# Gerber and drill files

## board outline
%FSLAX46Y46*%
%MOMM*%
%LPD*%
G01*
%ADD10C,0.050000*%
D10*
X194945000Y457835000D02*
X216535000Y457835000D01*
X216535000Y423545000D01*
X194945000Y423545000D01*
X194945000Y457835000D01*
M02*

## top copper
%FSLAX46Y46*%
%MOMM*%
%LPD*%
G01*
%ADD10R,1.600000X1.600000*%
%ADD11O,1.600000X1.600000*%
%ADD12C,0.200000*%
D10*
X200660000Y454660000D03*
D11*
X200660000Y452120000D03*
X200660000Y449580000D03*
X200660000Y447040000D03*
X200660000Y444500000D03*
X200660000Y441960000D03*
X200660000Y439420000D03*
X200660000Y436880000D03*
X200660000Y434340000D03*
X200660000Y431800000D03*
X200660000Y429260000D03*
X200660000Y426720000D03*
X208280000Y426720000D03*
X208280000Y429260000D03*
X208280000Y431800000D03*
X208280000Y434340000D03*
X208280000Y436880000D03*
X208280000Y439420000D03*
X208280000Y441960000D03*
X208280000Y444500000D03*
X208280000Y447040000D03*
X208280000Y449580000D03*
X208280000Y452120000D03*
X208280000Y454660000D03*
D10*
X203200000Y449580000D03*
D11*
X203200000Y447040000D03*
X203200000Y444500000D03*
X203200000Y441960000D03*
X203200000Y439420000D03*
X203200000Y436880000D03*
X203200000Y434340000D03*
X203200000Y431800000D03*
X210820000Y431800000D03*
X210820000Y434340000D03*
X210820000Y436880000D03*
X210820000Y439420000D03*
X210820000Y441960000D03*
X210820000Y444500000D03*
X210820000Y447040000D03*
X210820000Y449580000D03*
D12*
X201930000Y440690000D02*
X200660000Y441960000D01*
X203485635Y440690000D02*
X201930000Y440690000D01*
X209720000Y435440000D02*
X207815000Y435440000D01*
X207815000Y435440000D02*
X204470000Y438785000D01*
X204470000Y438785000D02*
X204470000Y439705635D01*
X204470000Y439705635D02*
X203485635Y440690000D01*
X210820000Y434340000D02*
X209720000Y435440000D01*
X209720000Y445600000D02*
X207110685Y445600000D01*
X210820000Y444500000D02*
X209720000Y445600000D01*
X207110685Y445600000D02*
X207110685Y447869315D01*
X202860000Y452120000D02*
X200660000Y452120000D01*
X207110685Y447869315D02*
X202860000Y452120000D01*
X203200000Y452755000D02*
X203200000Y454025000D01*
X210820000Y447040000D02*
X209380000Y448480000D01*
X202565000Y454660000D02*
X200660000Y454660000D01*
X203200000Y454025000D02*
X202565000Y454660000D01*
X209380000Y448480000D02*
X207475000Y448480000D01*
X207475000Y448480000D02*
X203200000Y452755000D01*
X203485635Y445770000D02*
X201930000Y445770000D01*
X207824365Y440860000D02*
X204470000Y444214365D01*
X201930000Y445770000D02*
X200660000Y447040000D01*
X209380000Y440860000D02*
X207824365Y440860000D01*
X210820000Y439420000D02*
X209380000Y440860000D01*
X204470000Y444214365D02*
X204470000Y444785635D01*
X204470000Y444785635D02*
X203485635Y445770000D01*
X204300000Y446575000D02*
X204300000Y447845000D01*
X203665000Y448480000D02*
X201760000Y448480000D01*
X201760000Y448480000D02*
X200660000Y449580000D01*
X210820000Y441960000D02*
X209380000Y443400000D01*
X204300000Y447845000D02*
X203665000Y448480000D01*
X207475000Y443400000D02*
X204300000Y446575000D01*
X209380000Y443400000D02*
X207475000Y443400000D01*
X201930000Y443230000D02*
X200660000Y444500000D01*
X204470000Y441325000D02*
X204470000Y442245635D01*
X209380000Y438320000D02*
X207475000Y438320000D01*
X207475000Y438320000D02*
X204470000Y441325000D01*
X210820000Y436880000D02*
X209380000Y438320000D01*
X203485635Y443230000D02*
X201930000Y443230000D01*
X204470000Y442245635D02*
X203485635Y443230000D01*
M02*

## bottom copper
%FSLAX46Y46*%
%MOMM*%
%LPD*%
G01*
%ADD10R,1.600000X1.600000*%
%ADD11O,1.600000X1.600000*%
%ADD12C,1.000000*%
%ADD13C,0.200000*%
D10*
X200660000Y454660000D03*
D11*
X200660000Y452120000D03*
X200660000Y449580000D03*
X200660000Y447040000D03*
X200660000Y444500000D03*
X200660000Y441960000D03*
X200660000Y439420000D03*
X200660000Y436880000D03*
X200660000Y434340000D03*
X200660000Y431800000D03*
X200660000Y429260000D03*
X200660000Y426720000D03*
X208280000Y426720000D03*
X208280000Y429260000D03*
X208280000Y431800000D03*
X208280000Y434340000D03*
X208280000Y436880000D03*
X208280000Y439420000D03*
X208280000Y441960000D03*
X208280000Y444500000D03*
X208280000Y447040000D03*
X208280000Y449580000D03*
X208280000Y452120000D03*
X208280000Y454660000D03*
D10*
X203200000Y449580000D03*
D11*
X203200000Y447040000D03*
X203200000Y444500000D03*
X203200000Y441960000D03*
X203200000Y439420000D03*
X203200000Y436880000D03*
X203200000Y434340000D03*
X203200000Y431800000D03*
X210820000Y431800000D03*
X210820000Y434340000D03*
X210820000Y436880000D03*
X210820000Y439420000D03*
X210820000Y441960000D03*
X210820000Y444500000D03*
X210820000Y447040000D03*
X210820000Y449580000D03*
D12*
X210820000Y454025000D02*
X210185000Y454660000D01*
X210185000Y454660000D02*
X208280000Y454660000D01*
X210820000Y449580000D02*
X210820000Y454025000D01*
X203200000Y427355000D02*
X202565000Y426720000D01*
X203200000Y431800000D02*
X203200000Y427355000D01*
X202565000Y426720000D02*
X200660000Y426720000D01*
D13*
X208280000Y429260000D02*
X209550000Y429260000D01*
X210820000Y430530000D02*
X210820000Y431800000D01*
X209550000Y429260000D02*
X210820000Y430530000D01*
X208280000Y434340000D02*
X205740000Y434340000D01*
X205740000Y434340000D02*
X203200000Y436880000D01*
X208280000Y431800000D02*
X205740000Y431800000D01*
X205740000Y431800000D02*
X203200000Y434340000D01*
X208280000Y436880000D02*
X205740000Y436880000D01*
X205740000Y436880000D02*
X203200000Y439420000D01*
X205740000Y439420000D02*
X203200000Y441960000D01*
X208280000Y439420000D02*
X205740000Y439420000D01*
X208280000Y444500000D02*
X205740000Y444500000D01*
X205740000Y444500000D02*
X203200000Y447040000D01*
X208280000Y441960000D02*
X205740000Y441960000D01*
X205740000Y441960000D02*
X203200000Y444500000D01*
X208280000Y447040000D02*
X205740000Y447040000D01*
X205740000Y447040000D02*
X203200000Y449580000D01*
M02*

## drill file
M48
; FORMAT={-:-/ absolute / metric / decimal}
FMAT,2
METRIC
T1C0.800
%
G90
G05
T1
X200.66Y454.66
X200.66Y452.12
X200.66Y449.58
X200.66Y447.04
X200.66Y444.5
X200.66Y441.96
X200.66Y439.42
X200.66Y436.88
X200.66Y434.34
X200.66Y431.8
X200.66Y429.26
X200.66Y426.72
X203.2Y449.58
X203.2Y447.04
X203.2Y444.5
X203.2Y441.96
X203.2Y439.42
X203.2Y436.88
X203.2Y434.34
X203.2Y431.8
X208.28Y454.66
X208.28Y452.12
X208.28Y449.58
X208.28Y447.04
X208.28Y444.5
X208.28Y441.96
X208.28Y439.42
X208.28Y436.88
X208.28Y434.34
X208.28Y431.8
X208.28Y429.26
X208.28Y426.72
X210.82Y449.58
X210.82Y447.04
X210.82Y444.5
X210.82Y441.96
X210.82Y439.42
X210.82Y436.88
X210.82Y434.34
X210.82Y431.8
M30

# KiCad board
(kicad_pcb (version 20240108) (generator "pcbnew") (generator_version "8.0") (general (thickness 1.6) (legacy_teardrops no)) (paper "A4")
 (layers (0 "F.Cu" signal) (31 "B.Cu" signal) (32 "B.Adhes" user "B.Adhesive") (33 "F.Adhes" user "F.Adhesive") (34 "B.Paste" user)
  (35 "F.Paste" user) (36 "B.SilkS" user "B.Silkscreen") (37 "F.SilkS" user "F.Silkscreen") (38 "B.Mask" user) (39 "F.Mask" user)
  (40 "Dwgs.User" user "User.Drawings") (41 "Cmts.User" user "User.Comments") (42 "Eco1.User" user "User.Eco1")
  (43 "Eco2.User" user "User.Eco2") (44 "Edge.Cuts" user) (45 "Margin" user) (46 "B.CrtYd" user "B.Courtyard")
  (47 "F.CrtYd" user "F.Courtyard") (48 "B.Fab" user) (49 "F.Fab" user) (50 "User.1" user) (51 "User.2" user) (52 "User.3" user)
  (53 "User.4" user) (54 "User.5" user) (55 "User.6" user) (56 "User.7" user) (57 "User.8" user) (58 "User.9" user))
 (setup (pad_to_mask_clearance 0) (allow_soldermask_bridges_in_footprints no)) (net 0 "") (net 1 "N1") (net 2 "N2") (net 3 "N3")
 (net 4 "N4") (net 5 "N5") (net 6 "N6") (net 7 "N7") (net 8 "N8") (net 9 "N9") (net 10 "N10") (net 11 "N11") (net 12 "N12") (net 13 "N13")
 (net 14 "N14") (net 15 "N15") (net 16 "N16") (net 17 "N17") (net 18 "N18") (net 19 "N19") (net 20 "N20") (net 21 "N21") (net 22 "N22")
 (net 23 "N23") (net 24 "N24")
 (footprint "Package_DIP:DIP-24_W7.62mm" (layer "F.Cu") (at 200.66 -454.66)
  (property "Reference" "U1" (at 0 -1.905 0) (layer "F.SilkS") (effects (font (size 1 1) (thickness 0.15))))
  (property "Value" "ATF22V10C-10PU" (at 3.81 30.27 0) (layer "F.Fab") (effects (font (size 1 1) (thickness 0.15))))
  (pad "1" thru_hole rect (at 0 0) (size 1.6 1.6) (drill 0.8) (layers "*.Cu" "*.Mask") (remove_unused_layers no) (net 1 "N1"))
  (pad "2" thru_hole oval (at 0 2.54) (size 1.6 1.6) (drill 0.8) (layers "*.Cu" "*.Mask") (remove_unused_layers no) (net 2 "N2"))
  (pad "3" thru_hole oval (at 0 5.08) (size 1.6 1.6) (drill 0.8) (layers "*.Cu" "*.Mask") (remove_unused_layers no) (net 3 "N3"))
  (pad "4" thru_hole oval (at 0 7.62) (size 1.6 1.6) (drill 0.8) (layers "*.Cu" "*.Mask") (remove_unused_layers no) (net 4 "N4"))
  (pad "5" thru_hole oval (at 0 10.16) (size 1.6 1.6) (drill 0.8) (layers "*.Cu" "*.Mask") (remove_unused_layers no) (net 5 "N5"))
  (pad "6" thru_hole oval (at 0 12.7) (size 1.6 1.6) (drill 0.8) (layers "*.Cu" "*.Mask") (remove_unused_layers no) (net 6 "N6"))
  (pad "7" thru_hole oval (at 0 15.24) (size 1.6 1.6) (drill 0.8) (layers "*.Cu" "*.Mask") (remove_unused_layers no) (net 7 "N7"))
  (pad "8" thru_hole oval (at 0 17.78) (size 1.6 1.6) (drill 0.8) (layers "*.Cu" "*.Mask") (remove_unused_layers no) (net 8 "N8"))
  (pad "9" thru_hole oval (at 0 20.32) (size 1.6 1.6) (drill 0.8) (layers "*.Cu" "*.Mask") (remove_unused_layers no) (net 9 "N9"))
  (pad "10" thru_hole oval (at 0 22.86) (size 1.6 1.6) (drill 0.8) (layers "*.Cu" "*.Mask") (remove_unused_layers no) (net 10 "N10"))
  (pad "11" thru_hole oval (at 0 25.4) (size 1.6 1.6) (drill 0.8) (layers "*.Cu" "*.Mask") (remove_unused_layers no) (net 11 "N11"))
  (pad "12" thru_hole oval (at 0 27.94) (size 1.6 1.6) (drill 0.8) (layers "*.Cu" "*.Mask") (remove_unused_layers no) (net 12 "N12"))
  (pad "13" thru_hole oval (at 7.62 27.94) (size 1.6 1.6) (drill 0.8) (layers "*.Cu" "*.Mask") (remove_unused_layers no) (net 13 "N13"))
  (pad "14" thru_hole oval (at 7.62 25.4) (size 1.6 1.6) (drill 0.8) (layers "*.Cu" "*.Mask") (remove_unused_layers no) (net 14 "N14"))
  (pad "15" thru_hole oval (at 7.62 22.86) (size 1.6 1.6) (drill 0.8) (layers "*.Cu" "*.Mask") (remove_unused_layers no) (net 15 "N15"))
  (pad "16" thru_hole oval (at 7.62 20.32) (size 1.6 1.6) (drill 0.8) (layers "*.Cu" "*.Mask") (remove_unused_layers no) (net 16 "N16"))
  (pad "17" thru_hole oval (at 7.62 17.78) (size 1.6 1.6) (drill 0.8) (layers "*.Cu" "*.Mask") (remove_unused_layers no) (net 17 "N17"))
  (pad "18" thru_hole oval (at 7.62 15.24) (size 1.6 1.6) (drill 0.8) (layers "*.Cu" "*.Mask") (remove_unused_layers no) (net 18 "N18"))
  (pad "19" thru_hole oval (at 7.62 12.7) (size 1.6 1.6) (drill 0.8) (layers "*.Cu" "*.Mask") (remove_unused_layers no) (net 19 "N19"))
  (pad "20" thru_hole oval (at 7.62 10.16) (size 1.6 1.6) (drill 0.8) (layers "*.Cu" "*.Mask") (remove_unused_layers no) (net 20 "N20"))
  (pad "21" thru_hole oval (at 7.62 7.62) (size 1.6 1.6) (drill 0.8) (layers "*.Cu" "*.Mask") (remove_unused_layers no) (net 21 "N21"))
  (pad "22" thru_hole oval (at 7.62 5.08) (size 1.6 1.6) (drill 0.8) (layers "*.Cu" "*.Mask") (remove_unused_layers no) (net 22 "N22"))
  (pad "23" thru_hole oval (at 7.62 2.54) (size 1.6 1.6) (drill 0.8) (layers "*.Cu" "*.Mask") (remove_unused_layers no) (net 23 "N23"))
  (pad "24" thru_hole oval (at 7.62 0) (size 1.6 1.6) (drill 0.8) (layers "*.Cu" "*.Mask") (remove_unused_layers no) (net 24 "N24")))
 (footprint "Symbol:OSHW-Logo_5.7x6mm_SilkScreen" (layer "F.Cu") (at 212.725 -427.355 90)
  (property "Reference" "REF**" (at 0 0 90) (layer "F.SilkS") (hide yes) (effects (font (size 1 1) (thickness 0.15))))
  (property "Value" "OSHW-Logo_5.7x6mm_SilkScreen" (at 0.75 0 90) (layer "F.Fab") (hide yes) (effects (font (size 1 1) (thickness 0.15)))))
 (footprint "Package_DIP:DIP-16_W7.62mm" (layer "F.Cu") (at 203.2 -449.58)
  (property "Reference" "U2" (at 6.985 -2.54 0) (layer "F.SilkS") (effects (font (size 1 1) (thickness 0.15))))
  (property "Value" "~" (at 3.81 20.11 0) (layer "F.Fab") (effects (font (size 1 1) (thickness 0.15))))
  (pad "1" thru_hole rect (at 0 0) (size 1.6 1.6) (drill 0.8) (layers "*.Cu" "*.Mask") (remove_unused_layers no) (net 21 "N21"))
  (pad "2" thru_hole oval (at 0 2.54) (size 1.6 1.6) (drill 0.8) (layers "*.Cu" "*.Mask") (remove_unused_layers no) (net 20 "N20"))
  (pad "3" thru_hole oval (at 0 5.08) (size 1.6 1.6) (drill 0.8) (layers "*.Cu" "*.Mask") (remove_unused_layers no) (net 19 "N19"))
  (pad "4" thru_hole oval (at 0 7.62) (size 1.6 1.6) (drill 0.8) (layers "*.Cu" "*.Mask") (remove_unused_layers no) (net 18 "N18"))
  (pad "5" thru_hole oval (at 0 10.16) (size 1.6 1.6) (drill 0.8) (layers "*.Cu" "*.Mask") (remove_unused_layers no) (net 17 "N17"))
  (pad "6" thru_hole oval (at 0 12.7) (size 1.6 1.6) (drill 0.8) (layers "*.Cu" "*.Mask") (remove_unused_layers no) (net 16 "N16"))
  (pad "7" thru_hole oval (at 0 15.24) (size 1.6 1.6) (drill 0.8) (layers "*.Cu" "*.Mask") (remove_unused_layers no) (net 15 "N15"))
  (pad "8" thru_hole oval (at 0 17.78) (size 1.6 1.6) (drill 0.8) (layers "*.Cu" "*.Mask") (remove_unused_layers no) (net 12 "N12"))
  (pad "9" thru_hole oval (at 7.62 17.78) (size 1.6 1.6) (drill 0.8) (layers "*.Cu" "*.Mask") (remove_unused_layers no) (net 14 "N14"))
  (pad "10" thru_hole oval (at 7.62 15.24) (size 1.6 1.6) (drill 0.8) (layers "*.Cu" "*.Mask") (remove_unused_layers no) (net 6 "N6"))
  (pad "11" thru_hole oval (at 7.62 12.7) (size 1.6 1.6) (drill 0.8) (layers "*.Cu" "*.Mask") (remove_unused_layers no) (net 5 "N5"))
  (pad "12" thru_hole oval (at 7.62 10.16) (size 1.6 1.6) (drill 0.8) (layers "*.Cu" "*.Mask") (remove_unused_layers no) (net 4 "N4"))
  (pad "13" thru_hole oval (at 7.62 7.62) (size 1.6 1.6) (drill 0.8) (layers "*.Cu" "*.Mask") (remove_unused_layers no) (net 3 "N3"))
  (pad "14" thru_hole oval (at 7.62 5.08) (size 1.6 1.6) (drill 0.8) (layers "*.Cu" "*.Mask") (remove_unused_layers no) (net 2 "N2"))
  (pad "15" thru_hole oval (at 7.62 2.54) (size 1.6 1.6) (drill 0.8) (layers "*.Cu" "*.Mask") (remove_unused_layers no) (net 1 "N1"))
  (pad "16" thru_hole oval (at 7.62 0) (size 1.6 1.6) (drill 0.8) (layers "*.Cu" "*.Mask") (remove_unused_layers no) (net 24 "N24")))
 (gr_rect (start 194.945 -457.835) (end 216.535 -423.545) (stroke (width 0.05) (type default)) (fill none) (layer "Edge.Cuts"))
 (segment (start 210.82 -454.025) (end 210.185 -454.66) (width 1) (layer "B.Cu") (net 24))
 (segment (start 210.185 -454.66) (end 208.28 -454.66) (width 1) (layer "B.Cu") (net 24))
 (segment (start 210.82 -449.58) (end 210.82 -454.025) (width 1) (layer "B.Cu") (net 24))
 (segment (start 203.2 -427.355) (end 202.565 -426.72) (width 1) (layer "B.Cu") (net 12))
 (segment (start 203.2 -431.8) (end 203.2 -427.355) (width 1) (layer "B.Cu") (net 12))
 (segment (start 202.565 -426.72) (end 200.66 -426.72) (width 1) (layer "B.Cu") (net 12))
 (segment (start 208.28 -429.26) (end 209.55 -429.26) (width 0.2) (layer "B.Cu") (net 14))
 (segment (start 210.82 -430.53) (end 210.82 -431.8) (width 0.2) (layer "B.Cu") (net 14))
 (segment (start 209.55 -429.26) (end 210.82 -430.53) (width 0.2) (layer "B.Cu") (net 14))
 (segment (start 208.28 -434.34) (end 205.74 -434.34) (width 0.2) (layer "B.Cu") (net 16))
 (segment (start 205.74 -434.34) (end 203.2 -436.88) (width 0.2) (layer "B.Cu") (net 16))
 (segment (start 208.28 -431.8) (end 205.74 -431.8) (width 0.2) (layer "B.Cu") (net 15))
 (segment (start 205.74 -431.8) (end 203.2 -434.34) (width 0.2) (layer "B.Cu") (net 15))
 (segment (start 208.28 -436.88) (end 205.74 -436.88) (width 0.2) (layer "B.Cu") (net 17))
 (segment (start 205.74 -436.88) (end 203.2 -439.42) (width 0.2) (layer "B.Cu") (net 17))
 (segment (start 205.74 -439.42) (end 203.2 -441.96) (width 0.2) (layer "B.Cu") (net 18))
 (segment (start 208.28 -439.42) (end 205.74 -439.42) (width 0.2) (layer "B.Cu") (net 18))
 (segment (start 208.28 -444.5) (end 205.74 -444.5) (width 0.2) (layer "B.Cu") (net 20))
 (segment (start 205.74 -444.5) (end 203.2 -447.04) (width 0.2) (layer "B.Cu") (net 20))
 (segment (start 208.28 -441.96) (end 205.74 -441.96) (width 0.2) (layer "B.Cu") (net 19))
 (segment (start 205.74 -441.96) (end 203.2 -444.5) (width 0.2) (layer "B.Cu") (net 19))
 (segment (start 208.28 -447.04) (end 205.74 -447.04) (width 0.2) (layer "B.Cu") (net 21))
 (segment (start 205.74 -447.04) (end 203.2 -449.58) (width 0.2) (layer "B.Cu") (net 21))
 (segment (start 201.93 -440.69) (end 200.66 -441.96) (width 0.2) (layer "F.Cu") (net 6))
 (segment (start 203.485635 -440.69) (end 201.93 -440.69) (width 0.2) (layer "F.Cu") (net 6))
 (segment (start 209.72 -435.44) (end 207.815 -435.44) (width 0.2) (layer "F.Cu") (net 6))
 (segment (start 207.815 -435.44) (end 204.47 -438.785) (width 0.2) (layer "F.Cu") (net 6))
 (segment (start 204.47 -438.785) (end 204.47 -439.705635) (width 0.2) (layer "F.Cu") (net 6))
 (segment (start 204.47 -439.705635) (end 203.485635 -440.69) (width 0.2) (layer "F.Cu") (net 6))
 (segment (start 210.82 -434.34) (end 209.72 -435.44) (width 0.2) (layer "F.Cu") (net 6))
 (segment (start 209.72 -445.6) (end 207.110685 -445.6) (width 0.2) (layer "F.Cu") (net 2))
 (segment (start 210.82 -444.5) (end 209.72 -445.6) (width 0.2) (layer "F.Cu") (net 2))
 (segment (start 207.110685 -445.6) (end 207.110685 -447.869315) (width 0.2) (layer "F.Cu") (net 2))
 (segment (start 202.86 -452.12) (end 200.66 -452.12) (width 0.2) (layer "F.Cu") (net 2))
 (segment (start 207.110685 -447.869315) (end 202.86 -452.12) (width 0.2) (layer "F.Cu") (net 2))
 (segment (start 203.2 -452.755) (end 203.2 -454.025) (width 0.2) (layer "F.Cu") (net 1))
 (segment (start 210.82 -447.04) (end 209.38 -448.48) (width 0.2) (layer "F.Cu") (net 1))
 (segment (start 202.565 -454.66) (end 200.66 -454.66) (width 0.2) (layer "F.Cu") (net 1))
 (segment (start 203.2 -454.025) (end 202.565 -454.66) (width 0.2) (layer "F.Cu") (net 1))
 (segment (start 209.38 -448.48) (end 207.475 -448.48) (width 0.2) (layer "F.Cu") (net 1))
 (segment (start 207.475 -448.48) (end 203.2 -452.755) (width 0.2) (layer "F.Cu") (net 1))
 (segment (start 203.485635 -445.77) (end 201.93 -445.77) (width 0.2) (layer "F.Cu") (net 4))
 (segment (start 207.824365 -440.86) (end 204.47 -444.214365) (width 0.2) (layer "F.Cu") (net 4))
 (segment (start 201.93 -445.77) (end 200.66 -447.04) (width 0.2) (layer "F.Cu") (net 4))
 (segment (start 209.38 -440.86) (end 207.824365 -440.86) (width 0.2) (layer "F.Cu") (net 4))
 (segment (start 210.82 -439.42) (end 209.38 -440.86) (width 0.2) (layer "F.Cu") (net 4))
 (segment (start 204.47 -444.214365) (end 204.47 -444.785635) (width 0.2) (layer "F.Cu") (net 4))
 (segment (start 204.47 -444.785635) (end 203.485635 -445.77) (width 0.2) (layer "F.Cu") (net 4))
 (segment (start 204.3 -446.575) (end 204.3 -447.845) (width 0.2) (layer "F.Cu") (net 3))
 (segment (start 203.665 -448.48) (end 201.76 -448.48) (width 0.2) (layer "F.Cu") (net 3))
 (segment (start 201.76 -448.48) (end 200.66 -449.58) (width 0.2) (layer "F.Cu") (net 3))
 (segment (start 210.82 -441.96) (end 209.38 -443.4) (width 0.2) (layer "F.Cu") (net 3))
 (segment (start 204.3 -447.845) (end 203.665 -448.48) (width 0.2) (layer "F.Cu") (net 3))
 (segment (start 207.475 -443.4) (end 204.3 -446.575) (width 0.2) (layer "F.Cu") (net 3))
 (segment (start 209.38 -443.4) (end 207.475 -443.4) (width 0.2) (layer "F.Cu") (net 3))
 (segment (start 201.93 -443.23) (end 200.66 -444.5) (width 0.2) (layer "F.Cu") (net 5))
 (segment (start 204.47 -441.325) (end 204.47 -442.245635) (width 0.2) (layer "F.Cu") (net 5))
 (segment (start 209.38 -438.32) (end 207.475 -438.32) (width 0.2) (layer "F.Cu") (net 5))
 (segment (start 207.475 -438.32) (end 204.47 -441.325) (width 0.2) (layer "F.Cu") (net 5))
 (segment (start 210.82 -436.88) (end 209.38 -438.32) (width 0.2) (layer "F.Cu") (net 5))
 (segment (start 203.485635 -443.23) (end 201.93 -443.23) (width 0.2) (layer "F.Cu") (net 5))
 (segment (start 204.47 -442.245635) (end 203.485635 -443.23) (width 0.2) (layer "F.Cu") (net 5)))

